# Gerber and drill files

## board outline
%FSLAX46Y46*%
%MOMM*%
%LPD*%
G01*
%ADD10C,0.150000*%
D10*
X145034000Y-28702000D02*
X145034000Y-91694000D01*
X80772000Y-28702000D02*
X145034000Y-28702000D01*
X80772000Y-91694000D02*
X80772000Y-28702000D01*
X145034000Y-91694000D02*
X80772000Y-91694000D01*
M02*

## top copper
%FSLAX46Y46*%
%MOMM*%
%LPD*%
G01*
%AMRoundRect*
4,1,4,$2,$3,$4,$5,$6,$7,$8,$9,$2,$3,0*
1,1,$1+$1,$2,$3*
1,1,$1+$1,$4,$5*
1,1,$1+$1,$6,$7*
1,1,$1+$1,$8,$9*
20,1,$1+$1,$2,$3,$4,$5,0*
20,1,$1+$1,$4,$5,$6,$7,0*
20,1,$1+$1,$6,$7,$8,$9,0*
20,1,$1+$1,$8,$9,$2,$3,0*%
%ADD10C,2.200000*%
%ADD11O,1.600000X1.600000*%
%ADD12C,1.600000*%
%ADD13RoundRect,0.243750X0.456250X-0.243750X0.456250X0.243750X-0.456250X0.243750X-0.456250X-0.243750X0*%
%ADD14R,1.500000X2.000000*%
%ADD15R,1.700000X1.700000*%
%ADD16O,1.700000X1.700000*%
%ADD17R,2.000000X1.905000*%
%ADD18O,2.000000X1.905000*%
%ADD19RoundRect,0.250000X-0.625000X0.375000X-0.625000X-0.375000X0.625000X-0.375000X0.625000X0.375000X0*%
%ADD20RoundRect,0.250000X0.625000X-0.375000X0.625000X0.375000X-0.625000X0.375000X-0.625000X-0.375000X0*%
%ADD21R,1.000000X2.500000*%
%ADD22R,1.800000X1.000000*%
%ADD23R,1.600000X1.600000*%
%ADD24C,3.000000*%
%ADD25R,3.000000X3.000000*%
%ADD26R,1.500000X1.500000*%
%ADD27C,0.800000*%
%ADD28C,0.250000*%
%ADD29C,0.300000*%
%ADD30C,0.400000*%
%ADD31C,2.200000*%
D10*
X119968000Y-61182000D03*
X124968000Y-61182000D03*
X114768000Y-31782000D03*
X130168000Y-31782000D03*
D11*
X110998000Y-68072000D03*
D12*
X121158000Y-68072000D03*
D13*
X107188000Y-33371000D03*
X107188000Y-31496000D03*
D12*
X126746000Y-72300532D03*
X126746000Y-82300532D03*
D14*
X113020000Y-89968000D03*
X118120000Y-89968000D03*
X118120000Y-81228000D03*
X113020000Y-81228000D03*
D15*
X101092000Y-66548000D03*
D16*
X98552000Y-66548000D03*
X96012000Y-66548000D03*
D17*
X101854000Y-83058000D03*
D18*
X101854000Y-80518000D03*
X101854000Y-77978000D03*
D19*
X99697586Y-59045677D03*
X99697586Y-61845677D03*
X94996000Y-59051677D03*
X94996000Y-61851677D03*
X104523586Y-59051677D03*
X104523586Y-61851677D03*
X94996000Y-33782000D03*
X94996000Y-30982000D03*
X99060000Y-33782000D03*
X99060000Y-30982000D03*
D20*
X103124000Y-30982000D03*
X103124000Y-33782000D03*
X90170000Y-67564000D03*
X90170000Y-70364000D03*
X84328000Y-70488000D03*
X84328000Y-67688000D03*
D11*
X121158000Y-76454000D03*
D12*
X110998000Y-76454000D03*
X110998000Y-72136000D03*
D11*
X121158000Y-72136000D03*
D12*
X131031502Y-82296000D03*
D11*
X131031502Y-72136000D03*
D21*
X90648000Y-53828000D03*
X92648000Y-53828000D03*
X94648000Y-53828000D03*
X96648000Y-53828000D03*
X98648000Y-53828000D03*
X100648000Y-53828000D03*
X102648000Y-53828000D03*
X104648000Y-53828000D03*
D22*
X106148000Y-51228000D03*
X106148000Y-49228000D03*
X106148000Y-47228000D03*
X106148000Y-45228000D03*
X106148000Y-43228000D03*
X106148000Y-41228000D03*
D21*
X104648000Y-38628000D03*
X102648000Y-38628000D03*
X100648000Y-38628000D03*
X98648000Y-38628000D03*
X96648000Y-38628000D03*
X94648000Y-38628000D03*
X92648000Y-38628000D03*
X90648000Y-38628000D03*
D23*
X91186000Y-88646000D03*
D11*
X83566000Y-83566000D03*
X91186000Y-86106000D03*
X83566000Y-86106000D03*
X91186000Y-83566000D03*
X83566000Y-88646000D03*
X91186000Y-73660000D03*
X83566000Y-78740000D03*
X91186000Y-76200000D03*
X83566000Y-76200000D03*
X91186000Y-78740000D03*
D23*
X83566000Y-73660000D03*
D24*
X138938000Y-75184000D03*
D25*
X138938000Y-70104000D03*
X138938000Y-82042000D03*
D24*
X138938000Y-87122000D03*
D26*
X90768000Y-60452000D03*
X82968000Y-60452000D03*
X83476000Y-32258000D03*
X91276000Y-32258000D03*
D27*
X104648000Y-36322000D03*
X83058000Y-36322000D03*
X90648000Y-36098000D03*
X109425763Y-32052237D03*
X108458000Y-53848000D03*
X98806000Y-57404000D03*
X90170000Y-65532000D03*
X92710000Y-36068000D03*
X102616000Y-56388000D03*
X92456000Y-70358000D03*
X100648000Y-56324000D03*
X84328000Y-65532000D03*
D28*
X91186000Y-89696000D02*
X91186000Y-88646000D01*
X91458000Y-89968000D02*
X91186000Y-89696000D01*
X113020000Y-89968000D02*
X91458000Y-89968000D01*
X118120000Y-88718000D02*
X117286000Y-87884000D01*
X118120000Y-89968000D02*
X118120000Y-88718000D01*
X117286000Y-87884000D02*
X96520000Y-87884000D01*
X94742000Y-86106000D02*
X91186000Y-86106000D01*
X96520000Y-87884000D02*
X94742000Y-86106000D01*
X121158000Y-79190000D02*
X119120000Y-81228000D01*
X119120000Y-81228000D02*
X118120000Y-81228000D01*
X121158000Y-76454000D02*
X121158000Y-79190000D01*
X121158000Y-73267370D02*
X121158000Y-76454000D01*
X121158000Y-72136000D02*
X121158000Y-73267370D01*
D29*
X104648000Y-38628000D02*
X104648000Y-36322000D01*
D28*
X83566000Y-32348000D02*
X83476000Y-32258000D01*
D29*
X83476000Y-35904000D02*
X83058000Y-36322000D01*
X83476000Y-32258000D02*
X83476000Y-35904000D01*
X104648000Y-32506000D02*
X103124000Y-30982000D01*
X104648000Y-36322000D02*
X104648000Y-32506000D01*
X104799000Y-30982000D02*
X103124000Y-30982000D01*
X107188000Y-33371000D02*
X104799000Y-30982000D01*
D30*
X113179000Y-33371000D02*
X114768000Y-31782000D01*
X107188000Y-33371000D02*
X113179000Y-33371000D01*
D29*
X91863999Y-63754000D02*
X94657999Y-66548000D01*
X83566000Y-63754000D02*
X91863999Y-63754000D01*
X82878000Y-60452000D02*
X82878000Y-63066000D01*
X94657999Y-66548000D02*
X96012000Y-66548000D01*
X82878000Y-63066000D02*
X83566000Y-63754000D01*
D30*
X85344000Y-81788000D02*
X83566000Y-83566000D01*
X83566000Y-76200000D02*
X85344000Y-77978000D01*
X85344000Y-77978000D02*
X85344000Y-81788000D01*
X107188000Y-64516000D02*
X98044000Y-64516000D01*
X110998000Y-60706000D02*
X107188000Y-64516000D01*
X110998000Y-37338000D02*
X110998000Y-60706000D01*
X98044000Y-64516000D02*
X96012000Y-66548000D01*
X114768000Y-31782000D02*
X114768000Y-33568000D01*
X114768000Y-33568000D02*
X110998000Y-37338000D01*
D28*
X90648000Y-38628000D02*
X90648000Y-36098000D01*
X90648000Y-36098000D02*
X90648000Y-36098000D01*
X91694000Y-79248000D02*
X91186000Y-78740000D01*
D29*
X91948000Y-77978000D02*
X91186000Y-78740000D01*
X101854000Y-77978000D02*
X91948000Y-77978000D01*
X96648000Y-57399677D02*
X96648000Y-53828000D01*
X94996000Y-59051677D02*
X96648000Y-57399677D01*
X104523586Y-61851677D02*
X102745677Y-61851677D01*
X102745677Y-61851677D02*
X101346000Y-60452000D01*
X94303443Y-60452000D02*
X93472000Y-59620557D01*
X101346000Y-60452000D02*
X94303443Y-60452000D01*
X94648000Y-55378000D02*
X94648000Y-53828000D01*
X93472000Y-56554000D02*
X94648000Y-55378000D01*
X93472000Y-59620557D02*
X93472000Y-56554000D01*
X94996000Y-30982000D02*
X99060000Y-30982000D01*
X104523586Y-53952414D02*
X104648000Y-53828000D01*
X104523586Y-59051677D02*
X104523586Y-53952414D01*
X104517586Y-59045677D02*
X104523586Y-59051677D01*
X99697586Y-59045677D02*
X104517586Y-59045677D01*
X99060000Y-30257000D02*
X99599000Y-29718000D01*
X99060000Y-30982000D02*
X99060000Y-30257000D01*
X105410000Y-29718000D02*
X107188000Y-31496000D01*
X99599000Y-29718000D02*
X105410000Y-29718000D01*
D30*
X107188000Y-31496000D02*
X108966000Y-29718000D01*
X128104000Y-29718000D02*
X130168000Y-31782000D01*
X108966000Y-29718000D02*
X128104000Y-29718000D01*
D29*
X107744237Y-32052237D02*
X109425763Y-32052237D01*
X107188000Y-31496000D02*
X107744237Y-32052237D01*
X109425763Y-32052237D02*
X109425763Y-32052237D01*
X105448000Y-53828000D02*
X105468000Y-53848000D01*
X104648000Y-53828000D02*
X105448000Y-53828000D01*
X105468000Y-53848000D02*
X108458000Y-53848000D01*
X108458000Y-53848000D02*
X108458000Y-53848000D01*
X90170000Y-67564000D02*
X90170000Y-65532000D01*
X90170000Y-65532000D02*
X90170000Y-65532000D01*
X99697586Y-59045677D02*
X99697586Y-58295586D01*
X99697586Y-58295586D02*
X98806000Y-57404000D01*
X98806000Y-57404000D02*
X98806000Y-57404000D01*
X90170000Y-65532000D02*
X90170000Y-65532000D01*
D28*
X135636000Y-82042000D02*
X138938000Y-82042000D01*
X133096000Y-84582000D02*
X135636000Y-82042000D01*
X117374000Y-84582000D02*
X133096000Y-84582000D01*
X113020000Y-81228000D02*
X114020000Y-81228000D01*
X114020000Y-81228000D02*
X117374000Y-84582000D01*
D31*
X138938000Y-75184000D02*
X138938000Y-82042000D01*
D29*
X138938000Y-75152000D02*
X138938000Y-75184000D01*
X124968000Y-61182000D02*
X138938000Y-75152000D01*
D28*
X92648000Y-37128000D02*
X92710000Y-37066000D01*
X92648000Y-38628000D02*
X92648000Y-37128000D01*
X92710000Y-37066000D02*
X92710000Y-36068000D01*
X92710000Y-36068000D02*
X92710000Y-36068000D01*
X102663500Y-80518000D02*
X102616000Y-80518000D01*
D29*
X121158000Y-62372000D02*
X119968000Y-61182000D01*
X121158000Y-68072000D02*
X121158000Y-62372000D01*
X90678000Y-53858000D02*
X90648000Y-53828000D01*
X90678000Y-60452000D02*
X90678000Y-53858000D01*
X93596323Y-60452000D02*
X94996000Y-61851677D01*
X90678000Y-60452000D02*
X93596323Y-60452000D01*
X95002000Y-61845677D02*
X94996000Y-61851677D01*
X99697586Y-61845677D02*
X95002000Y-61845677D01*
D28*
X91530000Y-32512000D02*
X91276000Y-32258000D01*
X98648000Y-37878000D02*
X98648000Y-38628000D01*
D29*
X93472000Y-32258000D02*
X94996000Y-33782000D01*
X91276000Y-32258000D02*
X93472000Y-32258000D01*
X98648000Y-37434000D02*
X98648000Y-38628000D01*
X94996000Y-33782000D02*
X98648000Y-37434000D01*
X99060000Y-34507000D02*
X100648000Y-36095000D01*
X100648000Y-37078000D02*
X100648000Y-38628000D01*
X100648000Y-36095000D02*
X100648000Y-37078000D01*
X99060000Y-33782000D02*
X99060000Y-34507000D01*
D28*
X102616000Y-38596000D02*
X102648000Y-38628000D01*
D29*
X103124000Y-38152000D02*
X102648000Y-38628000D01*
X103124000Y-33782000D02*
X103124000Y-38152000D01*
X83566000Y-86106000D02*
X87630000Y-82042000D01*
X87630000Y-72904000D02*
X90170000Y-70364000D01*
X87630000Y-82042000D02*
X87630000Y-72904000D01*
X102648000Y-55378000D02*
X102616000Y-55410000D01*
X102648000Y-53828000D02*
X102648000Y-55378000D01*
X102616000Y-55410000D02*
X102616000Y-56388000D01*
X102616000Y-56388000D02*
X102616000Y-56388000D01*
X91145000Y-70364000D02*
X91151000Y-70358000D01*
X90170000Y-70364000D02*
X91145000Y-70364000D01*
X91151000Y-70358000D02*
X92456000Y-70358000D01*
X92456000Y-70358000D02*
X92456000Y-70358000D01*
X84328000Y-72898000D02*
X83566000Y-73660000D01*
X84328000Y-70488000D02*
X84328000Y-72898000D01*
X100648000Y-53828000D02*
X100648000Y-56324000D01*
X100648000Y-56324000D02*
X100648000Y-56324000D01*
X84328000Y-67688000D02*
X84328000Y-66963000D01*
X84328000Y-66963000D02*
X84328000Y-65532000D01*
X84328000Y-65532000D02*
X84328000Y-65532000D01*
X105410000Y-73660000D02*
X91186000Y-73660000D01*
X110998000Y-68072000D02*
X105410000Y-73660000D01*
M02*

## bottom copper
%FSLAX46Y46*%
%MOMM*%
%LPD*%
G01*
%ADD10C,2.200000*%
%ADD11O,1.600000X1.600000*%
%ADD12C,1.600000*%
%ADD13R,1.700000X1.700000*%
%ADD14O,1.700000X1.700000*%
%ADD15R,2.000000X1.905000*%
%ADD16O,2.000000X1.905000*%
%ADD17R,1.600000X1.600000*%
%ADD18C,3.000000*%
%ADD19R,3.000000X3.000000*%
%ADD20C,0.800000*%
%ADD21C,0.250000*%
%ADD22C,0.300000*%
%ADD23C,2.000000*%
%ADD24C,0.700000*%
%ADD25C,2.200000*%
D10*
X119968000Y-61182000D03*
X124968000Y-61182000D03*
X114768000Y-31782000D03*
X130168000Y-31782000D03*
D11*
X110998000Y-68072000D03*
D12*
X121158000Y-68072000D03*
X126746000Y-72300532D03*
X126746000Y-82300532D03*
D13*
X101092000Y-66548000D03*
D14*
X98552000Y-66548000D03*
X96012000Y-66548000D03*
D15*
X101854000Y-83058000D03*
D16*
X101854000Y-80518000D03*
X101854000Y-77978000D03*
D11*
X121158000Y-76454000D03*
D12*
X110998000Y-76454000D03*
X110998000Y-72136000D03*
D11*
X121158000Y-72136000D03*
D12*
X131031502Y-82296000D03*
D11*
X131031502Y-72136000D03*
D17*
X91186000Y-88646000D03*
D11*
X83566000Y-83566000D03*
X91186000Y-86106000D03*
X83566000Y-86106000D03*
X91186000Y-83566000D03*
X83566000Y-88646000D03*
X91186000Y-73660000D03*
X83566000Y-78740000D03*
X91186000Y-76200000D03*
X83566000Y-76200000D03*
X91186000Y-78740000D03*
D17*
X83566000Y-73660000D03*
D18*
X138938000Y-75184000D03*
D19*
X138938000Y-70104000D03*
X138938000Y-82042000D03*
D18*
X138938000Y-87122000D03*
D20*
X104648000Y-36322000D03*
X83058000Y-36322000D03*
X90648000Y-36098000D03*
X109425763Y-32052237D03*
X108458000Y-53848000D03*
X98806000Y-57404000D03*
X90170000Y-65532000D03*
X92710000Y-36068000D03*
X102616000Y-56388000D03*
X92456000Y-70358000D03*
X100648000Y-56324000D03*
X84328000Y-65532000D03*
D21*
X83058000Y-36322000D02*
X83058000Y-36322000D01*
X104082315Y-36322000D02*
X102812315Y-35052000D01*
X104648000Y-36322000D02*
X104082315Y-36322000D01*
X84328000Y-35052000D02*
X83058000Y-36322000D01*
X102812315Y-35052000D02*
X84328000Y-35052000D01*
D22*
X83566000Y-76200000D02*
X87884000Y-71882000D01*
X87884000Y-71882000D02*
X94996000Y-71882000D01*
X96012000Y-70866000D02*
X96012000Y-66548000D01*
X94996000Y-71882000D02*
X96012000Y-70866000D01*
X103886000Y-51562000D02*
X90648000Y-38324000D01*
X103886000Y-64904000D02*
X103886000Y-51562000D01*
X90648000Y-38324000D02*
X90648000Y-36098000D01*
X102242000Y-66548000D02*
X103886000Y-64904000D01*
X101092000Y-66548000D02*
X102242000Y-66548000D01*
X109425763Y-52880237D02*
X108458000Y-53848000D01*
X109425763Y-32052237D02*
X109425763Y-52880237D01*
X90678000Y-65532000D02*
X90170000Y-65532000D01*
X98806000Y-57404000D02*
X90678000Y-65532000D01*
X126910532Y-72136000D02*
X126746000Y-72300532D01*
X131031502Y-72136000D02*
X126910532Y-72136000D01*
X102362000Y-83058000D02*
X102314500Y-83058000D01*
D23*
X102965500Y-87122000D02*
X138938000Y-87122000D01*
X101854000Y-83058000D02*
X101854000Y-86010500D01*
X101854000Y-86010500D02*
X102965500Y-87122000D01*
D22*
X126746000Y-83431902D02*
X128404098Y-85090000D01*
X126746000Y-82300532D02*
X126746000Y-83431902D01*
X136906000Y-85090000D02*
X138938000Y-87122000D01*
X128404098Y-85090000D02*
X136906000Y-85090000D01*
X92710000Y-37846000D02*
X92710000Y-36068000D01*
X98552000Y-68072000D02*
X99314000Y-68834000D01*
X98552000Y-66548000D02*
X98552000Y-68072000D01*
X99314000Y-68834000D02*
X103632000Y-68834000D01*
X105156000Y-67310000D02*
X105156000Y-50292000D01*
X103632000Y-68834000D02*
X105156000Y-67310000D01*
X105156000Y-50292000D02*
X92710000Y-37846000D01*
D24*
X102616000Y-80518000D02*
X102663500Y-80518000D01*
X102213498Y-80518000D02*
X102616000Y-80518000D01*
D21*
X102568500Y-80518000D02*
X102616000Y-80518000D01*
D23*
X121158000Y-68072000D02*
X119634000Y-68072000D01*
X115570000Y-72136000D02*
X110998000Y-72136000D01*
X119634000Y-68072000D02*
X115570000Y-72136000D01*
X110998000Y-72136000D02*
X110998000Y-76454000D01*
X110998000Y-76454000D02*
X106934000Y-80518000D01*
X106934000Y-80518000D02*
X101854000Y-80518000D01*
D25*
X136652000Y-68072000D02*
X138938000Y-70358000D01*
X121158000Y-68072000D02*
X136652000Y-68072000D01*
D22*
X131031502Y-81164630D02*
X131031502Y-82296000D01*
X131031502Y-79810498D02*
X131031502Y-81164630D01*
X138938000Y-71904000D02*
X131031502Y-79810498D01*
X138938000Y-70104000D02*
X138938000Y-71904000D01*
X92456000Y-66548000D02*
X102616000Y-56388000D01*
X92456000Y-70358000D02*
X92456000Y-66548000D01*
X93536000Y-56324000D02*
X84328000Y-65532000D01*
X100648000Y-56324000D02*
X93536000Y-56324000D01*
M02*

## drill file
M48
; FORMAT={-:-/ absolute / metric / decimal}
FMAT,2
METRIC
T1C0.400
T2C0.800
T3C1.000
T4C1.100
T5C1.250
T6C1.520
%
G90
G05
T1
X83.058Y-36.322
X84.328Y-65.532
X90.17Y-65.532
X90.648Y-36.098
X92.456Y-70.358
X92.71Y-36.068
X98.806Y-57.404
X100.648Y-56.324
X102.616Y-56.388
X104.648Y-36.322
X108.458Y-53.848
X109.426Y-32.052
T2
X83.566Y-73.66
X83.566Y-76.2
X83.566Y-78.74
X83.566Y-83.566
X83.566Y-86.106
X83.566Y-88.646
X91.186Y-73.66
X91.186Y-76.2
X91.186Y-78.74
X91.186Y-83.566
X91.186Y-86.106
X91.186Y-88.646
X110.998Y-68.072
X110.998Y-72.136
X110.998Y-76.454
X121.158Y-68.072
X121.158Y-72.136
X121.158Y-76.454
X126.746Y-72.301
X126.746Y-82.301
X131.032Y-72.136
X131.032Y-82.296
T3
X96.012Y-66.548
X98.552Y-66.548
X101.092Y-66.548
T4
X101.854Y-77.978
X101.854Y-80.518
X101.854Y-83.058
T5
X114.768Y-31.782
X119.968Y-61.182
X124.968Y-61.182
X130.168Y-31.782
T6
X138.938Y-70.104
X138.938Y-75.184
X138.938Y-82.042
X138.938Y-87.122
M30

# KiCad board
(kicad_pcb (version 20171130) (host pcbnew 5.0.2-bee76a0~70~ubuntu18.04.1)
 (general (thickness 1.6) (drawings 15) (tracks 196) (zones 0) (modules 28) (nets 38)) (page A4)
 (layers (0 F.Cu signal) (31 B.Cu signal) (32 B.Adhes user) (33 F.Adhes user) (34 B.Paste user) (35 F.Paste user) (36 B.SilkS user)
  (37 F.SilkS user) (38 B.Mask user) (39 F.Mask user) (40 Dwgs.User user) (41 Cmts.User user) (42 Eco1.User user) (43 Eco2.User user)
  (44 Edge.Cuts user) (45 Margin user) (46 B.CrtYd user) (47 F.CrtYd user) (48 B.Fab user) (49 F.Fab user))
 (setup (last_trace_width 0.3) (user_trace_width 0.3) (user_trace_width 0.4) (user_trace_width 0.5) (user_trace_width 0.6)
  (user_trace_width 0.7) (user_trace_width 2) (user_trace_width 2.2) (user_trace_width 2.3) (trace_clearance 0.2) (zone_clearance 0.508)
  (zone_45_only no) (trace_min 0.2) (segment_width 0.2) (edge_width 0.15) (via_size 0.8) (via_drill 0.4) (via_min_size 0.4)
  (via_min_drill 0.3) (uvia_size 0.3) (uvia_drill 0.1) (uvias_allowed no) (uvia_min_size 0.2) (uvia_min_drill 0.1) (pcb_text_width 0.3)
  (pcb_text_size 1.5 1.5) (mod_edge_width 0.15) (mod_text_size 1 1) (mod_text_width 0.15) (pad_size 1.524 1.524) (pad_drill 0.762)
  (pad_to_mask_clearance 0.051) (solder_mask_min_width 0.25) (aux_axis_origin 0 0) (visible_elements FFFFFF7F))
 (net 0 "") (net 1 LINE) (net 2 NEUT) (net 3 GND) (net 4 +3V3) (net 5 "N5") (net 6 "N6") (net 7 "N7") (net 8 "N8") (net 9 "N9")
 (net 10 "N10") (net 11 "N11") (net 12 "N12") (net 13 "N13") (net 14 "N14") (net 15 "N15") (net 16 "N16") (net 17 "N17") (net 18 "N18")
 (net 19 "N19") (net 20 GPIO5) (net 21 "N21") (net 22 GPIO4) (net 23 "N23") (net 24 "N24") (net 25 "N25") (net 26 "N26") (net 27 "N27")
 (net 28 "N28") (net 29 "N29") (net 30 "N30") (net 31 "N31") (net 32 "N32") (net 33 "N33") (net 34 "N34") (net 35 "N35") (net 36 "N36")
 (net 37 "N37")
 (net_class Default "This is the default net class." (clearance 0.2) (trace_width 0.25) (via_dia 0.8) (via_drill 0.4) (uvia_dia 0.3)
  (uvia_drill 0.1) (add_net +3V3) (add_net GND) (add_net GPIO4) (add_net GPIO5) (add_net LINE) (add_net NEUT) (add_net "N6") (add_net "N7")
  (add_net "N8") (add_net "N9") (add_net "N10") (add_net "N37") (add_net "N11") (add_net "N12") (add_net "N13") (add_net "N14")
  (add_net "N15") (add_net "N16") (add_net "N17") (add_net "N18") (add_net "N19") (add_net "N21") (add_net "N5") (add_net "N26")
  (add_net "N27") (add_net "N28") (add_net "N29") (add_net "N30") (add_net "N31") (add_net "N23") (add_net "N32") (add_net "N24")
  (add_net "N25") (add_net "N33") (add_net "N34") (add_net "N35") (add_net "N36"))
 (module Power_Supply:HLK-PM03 (layer F.Cu) (at 122.468 46.482 90)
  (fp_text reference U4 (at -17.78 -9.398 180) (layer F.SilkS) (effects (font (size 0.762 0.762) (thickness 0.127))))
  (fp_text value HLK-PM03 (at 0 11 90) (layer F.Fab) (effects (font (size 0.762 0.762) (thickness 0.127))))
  (pad 1 thru_hole circle (at -14.7 -2.5 90) (size 2.2 2.2) (drill 1.25) (layers *.Cu *.Mask) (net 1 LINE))
  (pad 2 thru_hole circle (at -14.7 2.5 90) (size 2.2 2.2) (drill 1.25) (layers *.Cu *.Mask) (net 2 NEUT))
  (pad 3 thru_hole circle (at 14.7 -7.7 90) (size 2.2 2.2) (drill 1.25) (layers *.Cu *.Mask) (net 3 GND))
  (pad 4 thru_hole circle (at 14.7 7.7 90) (size 2.2 2.2) (drill 1.25) (layers *.Cu *.Mask) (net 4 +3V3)))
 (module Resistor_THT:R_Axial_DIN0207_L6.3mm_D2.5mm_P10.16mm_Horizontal (layer F.Cu) (at 121.158 68.072 180)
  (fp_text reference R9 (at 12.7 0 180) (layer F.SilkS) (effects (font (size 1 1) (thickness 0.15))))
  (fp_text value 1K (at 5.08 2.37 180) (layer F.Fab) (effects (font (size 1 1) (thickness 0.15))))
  (pad 2 thru_hole oval (at 10.16 0 180) (size 1.6 1.6) (drill 0.8) (layers *.Cu *.Mask) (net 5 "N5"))
  (pad 1 thru_hole circle (at 0 0 180) (size 1.6 1.6) (drill 0.8) (layers *.Cu *.Mask) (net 1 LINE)))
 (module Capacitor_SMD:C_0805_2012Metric (layer F.Cu) (at 107.188 32.4335 90)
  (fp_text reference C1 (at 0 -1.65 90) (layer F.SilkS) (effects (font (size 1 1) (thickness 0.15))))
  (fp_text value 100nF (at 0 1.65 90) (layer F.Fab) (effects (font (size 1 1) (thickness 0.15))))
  (pad 1 smd roundrect (at -0.9375 0 90) (size 0.975 1.4) (layers F.Cu F.Paste F.Mask) (roundrect_rratio 0.25) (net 3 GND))
  (pad 2 smd roundrect (at 0.9375 0 90) (size 0.975 1.4) (layers F.Cu F.Paste F.Mask) (roundrect_rratio 0.25) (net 4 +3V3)))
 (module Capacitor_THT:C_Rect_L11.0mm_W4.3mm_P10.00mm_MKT (layer F.Cu) (at 126.746 72.300532 270)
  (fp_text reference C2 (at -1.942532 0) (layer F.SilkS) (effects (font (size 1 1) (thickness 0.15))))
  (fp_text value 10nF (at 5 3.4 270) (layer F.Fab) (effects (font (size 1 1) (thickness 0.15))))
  (pad 1 thru_hole circle (at 0 0 270) (size 1.6 1.6) (drill 0.8) (layers *.Cu *.Mask) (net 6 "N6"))
  (pad 2 thru_hole circle (at 10 0 270) (size 1.6 1.6) (drill 0.8) (layers *.Cu *.Mask) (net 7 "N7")))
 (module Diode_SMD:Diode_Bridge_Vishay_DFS (layer F.Cu) (at 115.57 85.598 90)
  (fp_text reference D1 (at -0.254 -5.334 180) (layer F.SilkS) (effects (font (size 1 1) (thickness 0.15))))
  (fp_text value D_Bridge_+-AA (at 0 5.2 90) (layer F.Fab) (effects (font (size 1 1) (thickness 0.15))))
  (pad 1 smd rect (at -4.37 -2.55 90) (size 2 1.5) (layers F.Cu F.Paste F.Mask) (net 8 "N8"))
  (pad 2 smd rect (at -4.37 2.55 90) (size 2 1.5) (layers F.Cu F.Paste F.Mask) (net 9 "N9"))
  (pad 3 smd rect (at 4.37 2.55 90) (size 2 1.5) (layers F.Cu F.Paste F.Mask) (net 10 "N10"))
  (pad 4 smd rect (at 4.37 -2.55 90) (size 2 1.5) (layers F.Cu F.Paste F.Mask) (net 2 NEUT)))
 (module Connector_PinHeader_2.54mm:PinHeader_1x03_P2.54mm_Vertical (layer F.Cu) (at 101.092 66.548 270)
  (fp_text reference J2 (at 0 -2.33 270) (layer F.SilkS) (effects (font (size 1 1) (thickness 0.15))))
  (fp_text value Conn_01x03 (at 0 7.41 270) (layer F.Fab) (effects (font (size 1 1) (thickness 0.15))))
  (pad 1 thru_hole rect (at 0 0 270) (size 1.7 1.7) (drill 1) (layers *.Cu *.Mask) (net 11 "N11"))
  (pad 2 thru_hole oval (at 0 2.54 270) (size 1.7 1.7) (drill 1) (layers *.Cu *.Mask) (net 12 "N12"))
  (pad 3 thru_hole oval (at 0 5.08 270) (size 1.7 1.7) (drill 1) (layers *.Cu *.Mask) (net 3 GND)))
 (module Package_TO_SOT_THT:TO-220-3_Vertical (layer F.Cu) (at 101.854 83.058 90)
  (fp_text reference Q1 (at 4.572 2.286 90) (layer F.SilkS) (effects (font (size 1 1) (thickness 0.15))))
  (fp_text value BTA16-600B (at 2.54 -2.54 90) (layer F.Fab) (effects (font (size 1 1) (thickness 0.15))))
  (pad 1 thru_hole rect (at 0 0 90) (size 1.905 2) (drill 1.1) (layers *.Cu *.Mask) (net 7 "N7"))
  (pad 2 thru_hole oval (at 2.54 0 90) (size 1.905 2) (drill 1.1) (layers *.Cu *.Mask) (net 1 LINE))
  (pad 3 thru_hole oval (at 5.08 0 90) (size 1.905 2) (drill 1.1) (layers *.Cu *.Mask) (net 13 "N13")))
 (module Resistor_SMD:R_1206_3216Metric (layer F.Cu) (at 99.697586 60.445677 270)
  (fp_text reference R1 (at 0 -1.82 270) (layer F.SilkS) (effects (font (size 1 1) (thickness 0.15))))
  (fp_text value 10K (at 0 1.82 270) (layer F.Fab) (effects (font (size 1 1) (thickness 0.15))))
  (pad 1 smd roundrect (at -1.4 0 270) (size 1.25 1.75) (layers F.Cu F.Paste F.Mask) (roundrect_rratio 0.2) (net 4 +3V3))
  (pad 2 smd roundrect (at 1.4 0 270) (size 1.25 1.75) (layers F.Cu F.Paste F.Mask) (roundrect_rratio 0.2) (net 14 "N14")))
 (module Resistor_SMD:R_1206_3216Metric (layer F.Cu) (at 94.996 60.451677 270)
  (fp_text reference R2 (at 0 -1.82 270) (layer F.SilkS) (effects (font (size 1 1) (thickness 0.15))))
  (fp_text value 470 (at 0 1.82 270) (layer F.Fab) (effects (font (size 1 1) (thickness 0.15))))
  (pad 1 smd roundrect (at -1.4 0 270) (size 1.25 1.75) (layers F.Cu F.Paste F.Mask) (roundrect_rratio 0.2) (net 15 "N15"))
  (pad 2 smd roundrect (at 1.4 0 270) (size 1.25 1.75) (layers F.Cu F.Paste F.Mask) (roundrect_rratio 0.2) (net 14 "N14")))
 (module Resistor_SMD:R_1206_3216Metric (layer F.Cu) (at 104.523586 60.451677 270)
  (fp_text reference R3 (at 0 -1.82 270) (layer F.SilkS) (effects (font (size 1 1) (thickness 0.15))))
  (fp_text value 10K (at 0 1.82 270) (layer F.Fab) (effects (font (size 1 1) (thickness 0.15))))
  (pad 1 smd roundrect (at -1.4 0 270) (size 1.25 1.75) (layers F.Cu F.Paste F.Mask) (roundrect_rratio 0.2) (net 4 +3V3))
  (pad 2 smd roundrect (at 1.4 0 270) (size 1.25 1.75) (layers F.Cu F.Paste F.Mask) (roundrect_rratio 0.2) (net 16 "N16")))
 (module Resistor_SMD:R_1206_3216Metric (layer F.Cu) (at 94.996 32.382 270)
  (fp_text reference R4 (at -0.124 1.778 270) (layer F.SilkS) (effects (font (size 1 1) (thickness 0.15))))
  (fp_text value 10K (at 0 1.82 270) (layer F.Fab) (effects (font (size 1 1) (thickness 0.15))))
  (pad 2 smd roundrect (at 1.4 0 270) (size 1.25 1.75) (layers F.Cu F.Paste F.Mask) (roundrect_rratio 0.2) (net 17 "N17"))
  (pad 1 smd roundrect (at -1.4 0 270) (size 1.25 1.75) (layers F.Cu F.Paste F.Mask) (roundrect_rratio 0.2) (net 4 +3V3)))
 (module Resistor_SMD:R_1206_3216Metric (layer F.Cu) (at 99.06 32.382 270)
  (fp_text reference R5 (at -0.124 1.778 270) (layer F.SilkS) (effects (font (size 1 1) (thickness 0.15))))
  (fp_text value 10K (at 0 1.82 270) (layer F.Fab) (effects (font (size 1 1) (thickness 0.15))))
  (pad 2 smd roundrect (at 1.4 0 270) (size 1.25 1.75) (layers F.Cu F.Paste F.Mask) (roundrect_rratio 0.2) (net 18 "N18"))
  (pad 1 smd roundrect (at -1.4 0 270) (size 1.25 1.75) (layers F.Cu F.Paste F.Mask) (roundrect_rratio 0.2) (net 4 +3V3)))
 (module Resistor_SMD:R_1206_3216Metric (layer F.Cu) (at 103.124 32.382 90)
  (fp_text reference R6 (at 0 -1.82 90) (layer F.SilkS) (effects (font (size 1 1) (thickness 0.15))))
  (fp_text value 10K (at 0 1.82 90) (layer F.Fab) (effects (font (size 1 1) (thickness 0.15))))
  (pad 2 smd roundrect (at 1.4 0 90) (size 1.25 1.75) (layers F.Cu F.Paste F.Mask) (roundrect_rratio 0.2) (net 3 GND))
  (pad 1 smd roundrect (at -1.4 0 90) (size 1.25 1.75) (layers F.Cu F.Paste F.Mask) (roundrect_rratio 0.2) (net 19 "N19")))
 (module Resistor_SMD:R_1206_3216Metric (layer F.Cu) (at 90.17 68.964 90)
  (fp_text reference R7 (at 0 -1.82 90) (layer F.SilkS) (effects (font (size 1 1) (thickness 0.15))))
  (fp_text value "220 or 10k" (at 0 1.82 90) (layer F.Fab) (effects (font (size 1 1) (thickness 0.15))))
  (pad 2 smd roundrect (at 1.4 0 90) (size 1.25 1.75) (layers F.Cu F.Paste F.Mask) (roundrect_rratio 0.2) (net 4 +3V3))
  (pad 1 smd roundrect (at -1.4 0 90) (size 1.25 1.75) (layers F.Cu F.Paste F.Mask) (roundrect_rratio 0.2) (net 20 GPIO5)))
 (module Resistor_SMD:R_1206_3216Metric (layer F.Cu) (at 84.328 69.088 90)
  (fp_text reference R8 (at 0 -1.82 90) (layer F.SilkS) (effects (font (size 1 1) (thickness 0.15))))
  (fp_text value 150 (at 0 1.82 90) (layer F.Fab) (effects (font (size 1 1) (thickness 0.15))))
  (pad 1 smd roundrect (at -1.4 0 90) (size 1.25 1.75) (layers F.Cu F.Paste F.Mask) (roundrect_rratio 0.2) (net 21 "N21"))
  (pad 2 smd roundrect (at 1.4 0 90) (size 1.25 1.75) (layers F.Cu F.Paste F.Mask) (roundrect_rratio 0.2) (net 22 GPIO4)))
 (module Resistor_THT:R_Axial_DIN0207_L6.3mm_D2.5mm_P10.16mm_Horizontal (layer F.Cu) (at 110.998 76.454)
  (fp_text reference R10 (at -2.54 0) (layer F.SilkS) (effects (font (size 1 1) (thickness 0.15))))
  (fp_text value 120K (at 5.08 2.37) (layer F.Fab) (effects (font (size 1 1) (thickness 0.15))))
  (pad 2 thru_hole oval (at 10.16 0) (size 1.6 1.6) (drill 0.8) (layers *.Cu *.Mask) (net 10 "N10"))
  (pad 1 thru_hole circle (at 0 0) (size 1.6 1.6) (drill 0.8) (layers *.Cu *.Mask) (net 1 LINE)))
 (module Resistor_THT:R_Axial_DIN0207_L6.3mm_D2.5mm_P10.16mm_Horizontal (layer F.Cu) (at 110.998 72.136)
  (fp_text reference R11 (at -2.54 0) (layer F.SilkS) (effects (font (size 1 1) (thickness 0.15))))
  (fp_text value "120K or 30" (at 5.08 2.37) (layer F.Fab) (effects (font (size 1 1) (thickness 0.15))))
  (pad 1 thru_hole circle (at 0 0) (size 1.6 1.6) (drill 0.8) (layers *.Cu *.Mask) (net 1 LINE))
  (pad 2 thru_hole oval (at 10.16 0) (size 1.6 1.6) (drill 0.8) (layers *.Cu *.Mask) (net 10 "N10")))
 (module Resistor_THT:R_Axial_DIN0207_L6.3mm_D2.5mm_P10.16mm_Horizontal (layer F.Cu) (at 131.031502 82.296 90)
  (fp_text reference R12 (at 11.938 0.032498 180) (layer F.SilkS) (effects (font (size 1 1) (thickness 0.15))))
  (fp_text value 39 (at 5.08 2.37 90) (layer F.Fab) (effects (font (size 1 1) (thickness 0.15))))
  (pad 1 thru_hole circle (at 0 0 90) (size 1.6 1.6) (drill 0.8) (layers *.Cu *.Mask) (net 1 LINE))
  (pad 2 thru_hole oval (at 10.16 0 90) (size 1.6 1.6) (drill 0.8) (layers *.Cu *.Mask) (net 6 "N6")))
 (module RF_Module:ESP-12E (layer F.Cu) (at 94.148 46.228 90)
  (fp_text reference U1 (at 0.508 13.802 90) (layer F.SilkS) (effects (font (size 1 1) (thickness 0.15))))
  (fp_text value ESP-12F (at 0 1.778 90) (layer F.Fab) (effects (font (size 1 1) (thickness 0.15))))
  (pad 1 smd rect (at -7.6 -3.5 90) (size 2.5 1) (layers F.Cu F.Paste F.Mask) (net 14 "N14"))
  (pad 2 smd rect (at -7.6 -1.5 90) (size 2.5 1) (layers F.Cu F.Paste F.Mask) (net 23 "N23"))
  (pad 3 smd rect (at -7.6 0.5 90) (size 2.5 1) (layers F.Cu F.Paste F.Mask) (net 16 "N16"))
  (pad 4 smd rect (at -7.6 2.5 90) (size 2.5 1) (layers F.Cu F.Paste F.Mask) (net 15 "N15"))
  (pad 5 smd rect (at -7.6 4.5 90) (size 2.5 1) (layers F.Cu F.Paste F.Mask) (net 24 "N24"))
  (pad 6 smd rect (at -7.6 6.5 90) (size 2.5 1) (layers F.Cu F.Paste F.Mask) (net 22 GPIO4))
  (pad 7 smd rect (at -7.6 8.5 90) (size 2.5 1) (layers F.Cu F.Paste F.Mask) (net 20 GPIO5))
  (pad 8 smd rect (at -7.6 10.5 90) (size 2.5 1) (layers F.Cu F.Paste F.Mask) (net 4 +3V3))
  (pad 9 smd rect (at -5 12 90) (size 1 1.8) (layers F.Cu F.Paste F.Mask) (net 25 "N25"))
  (pad 10 smd rect (at -3 12 90) (size 1 1.8) (layers F.Cu F.Paste F.Mask) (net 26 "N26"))
  (pad 11 smd rect (at -1 12 90) (size 1 1.8) (layers F.Cu F.Paste F.Mask) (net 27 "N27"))
  (pad 12 smd rect (at 1 12 90) (size 1 1.8) (layers F.Cu F.Paste F.Mask) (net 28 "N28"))
  (pad 13 smd rect (at 3 12 90) (size 1 1.8) (layers F.Cu F.Paste F.Mask) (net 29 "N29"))
  (pad 14 smd rect (at 5 12 90) (size 1 1.8) (layers F.Cu F.Paste F.Mask) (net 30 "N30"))
  (pad 15 smd rect (at 7.6 10.5 90) (size 2.5 1) (layers F.Cu F.Paste F.Mask) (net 3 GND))
  (pad 16 smd rect (at 7.6 8.5 90) (size 2.5 1) (layers F.Cu F.Paste F.Mask) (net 19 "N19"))
  (pad 17 smd rect (at 7.6 6.5 90) (size 2.5 1) (layers F.Cu F.Paste F.Mask) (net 18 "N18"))
  (pad 18 smd rect (at 7.6 4.5 90) (size 2.5 1) (layers F.Cu F.Paste F.Mask) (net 17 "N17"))
  (pad 19 smd rect (at 7.6 2.5 90) (size 2.5 1) (layers F.Cu F.Paste F.Mask) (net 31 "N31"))
  (pad 20 smd rect (at 7.6 0.5 90) (size 2.5 1) (layers F.Cu F.Paste F.Mask) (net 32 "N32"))
  (pad 21 smd rect (at 7.6 -1.5 90) (size 2.5 1) (layers F.Cu F.Paste F.Mask) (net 12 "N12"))
  (pad 22 smd rect (at 7.6 -3.5 90) (size 2.5 1) (layers F.Cu F.Paste F.Mask) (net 11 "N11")))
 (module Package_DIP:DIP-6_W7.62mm (layer F.Cu) (at 91.186 88.646 180)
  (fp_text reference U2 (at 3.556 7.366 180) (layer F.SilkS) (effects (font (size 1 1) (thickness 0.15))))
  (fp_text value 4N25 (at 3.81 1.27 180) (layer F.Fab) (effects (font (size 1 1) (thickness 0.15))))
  (pad 1 thru_hole rect (at 0 0 180) (size 1.6 1.6) (drill 0.8) (layers *.Cu *.Mask) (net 8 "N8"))
  (pad 4 thru_hole oval (at 7.62 5.08 180) (size 1.6 1.6) (drill 0.8) (layers *.Cu *.Mask) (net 3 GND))
  (pad 2 thru_hole oval (at 0 2.54 180) (size 1.6 1.6) (drill 0.8) (layers *.Cu *.Mask) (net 9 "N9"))
  (pad 5 thru_hole oval (at 7.62 2.54 180) (size 1.6 1.6) (drill 0.8) (layers *.Cu *.Mask) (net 20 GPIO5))
  (pad 3 thru_hole oval (at 0 5.08 180) (size 1.6 1.6) (drill 0.8) (layers *.Cu *.Mask) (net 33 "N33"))
  (pad 6 thru_hole oval (at 7.62 0 180) (size 1.6 1.6) (drill 0.8) (layers *.Cu *.Mask) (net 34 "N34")))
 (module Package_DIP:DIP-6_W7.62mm (layer F.Cu) (at 83.566 73.66)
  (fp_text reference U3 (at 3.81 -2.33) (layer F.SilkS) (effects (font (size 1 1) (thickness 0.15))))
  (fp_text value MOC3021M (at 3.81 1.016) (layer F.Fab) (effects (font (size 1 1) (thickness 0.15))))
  (pad 6 thru_hole oval (at 7.62 0) (size 1.6 1.6) (drill 0.8) (layers *.Cu *.Mask) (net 5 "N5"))
  (pad 3 thru_hole oval (at 0 5.08) (size 1.6 1.6) (drill 0.8) (layers *.Cu *.Mask) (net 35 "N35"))
  (pad 5 thru_hole oval (at 7.62 2.54) (size 1.6 1.6) (drill 0.8) (layers *.Cu *.Mask) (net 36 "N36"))
  (pad 2 thru_hole oval (at 0 2.54) (size 1.6 1.6) (drill 0.8) (layers *.Cu *.Mask) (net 3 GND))
  (pad 4 thru_hole oval (at 7.62 5.08) (size 1.6 1.6) (drill 0.8) (layers *.Cu *.Mask) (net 13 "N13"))
  (pad 1 thru_hole rect (at 0 0) (size 1.6 1.6) (drill 0.8) (layers *.Cu *.Mask) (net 21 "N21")))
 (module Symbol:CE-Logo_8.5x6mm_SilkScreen (layer F.Cu) (at 126.238 87.63)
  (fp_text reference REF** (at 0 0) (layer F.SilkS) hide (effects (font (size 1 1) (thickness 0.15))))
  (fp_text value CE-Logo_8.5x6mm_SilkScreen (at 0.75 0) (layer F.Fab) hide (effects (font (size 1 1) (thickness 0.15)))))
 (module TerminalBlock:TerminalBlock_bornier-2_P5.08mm (layer F.Cu) (at 138.938 70.104 270)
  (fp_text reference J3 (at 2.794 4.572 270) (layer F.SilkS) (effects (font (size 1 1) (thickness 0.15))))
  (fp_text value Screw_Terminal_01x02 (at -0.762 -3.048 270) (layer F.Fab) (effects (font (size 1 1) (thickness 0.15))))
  (pad 2 thru_hole circle (at 5.08 0 270) (size 3 3) (drill 1.52) (layers *.Cu *.Mask) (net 2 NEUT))
  (pad 1 thru_hole rect (at 0 0 270) (size 3 3) (drill 1.52) (layers *.Cu *.Mask) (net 1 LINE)))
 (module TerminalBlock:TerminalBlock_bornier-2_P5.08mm (layer F.Cu) (at 138.938 82.042 270)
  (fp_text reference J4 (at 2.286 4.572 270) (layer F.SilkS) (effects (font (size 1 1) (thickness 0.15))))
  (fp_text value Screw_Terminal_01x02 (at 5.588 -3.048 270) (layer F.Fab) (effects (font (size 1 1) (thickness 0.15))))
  (pad 1 thru_hole rect (at 0 0 270) (size 3 3) (drill 1.52) (layers *.Cu *.Mask) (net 2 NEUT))
  (pad 2 thru_hole circle (at 5.08 0 270) (size 3 3) (drill 1.52) (layers *.Cu *.Mask) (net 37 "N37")))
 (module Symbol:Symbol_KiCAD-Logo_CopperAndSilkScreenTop (layer F.Cu) (at 142.494 48.26 90)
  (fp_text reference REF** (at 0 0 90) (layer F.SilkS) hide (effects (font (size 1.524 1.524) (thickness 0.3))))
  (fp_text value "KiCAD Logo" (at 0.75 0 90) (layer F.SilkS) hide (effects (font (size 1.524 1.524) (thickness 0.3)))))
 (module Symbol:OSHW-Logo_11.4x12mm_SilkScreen (layer F.Cu) (at 138.684 35.56 90)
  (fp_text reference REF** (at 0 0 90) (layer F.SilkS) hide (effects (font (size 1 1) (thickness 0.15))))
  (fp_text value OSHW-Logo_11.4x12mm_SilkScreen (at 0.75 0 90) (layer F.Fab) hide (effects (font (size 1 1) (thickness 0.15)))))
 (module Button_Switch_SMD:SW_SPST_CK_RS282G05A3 (layer F.Cu) (at 86.868 60.452)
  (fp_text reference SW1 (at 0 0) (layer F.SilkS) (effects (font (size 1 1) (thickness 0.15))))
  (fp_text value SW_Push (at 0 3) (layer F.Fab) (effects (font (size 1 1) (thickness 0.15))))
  (pad 2 smd rect (at 3.9 0) (size 1.5 1.5) (layers F.Cu F.Paste F.Mask) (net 14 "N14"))
  (pad 1 smd rect (at -3.9 0) (size 1.5 1.5) (layers F.Cu F.Paste F.Mask) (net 3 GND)))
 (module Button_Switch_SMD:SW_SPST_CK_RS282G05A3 (layer F.Cu) (at 87.376 32.258)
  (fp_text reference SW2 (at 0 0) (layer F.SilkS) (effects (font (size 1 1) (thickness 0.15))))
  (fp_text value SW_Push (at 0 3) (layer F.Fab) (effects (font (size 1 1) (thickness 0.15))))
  (pad 1 smd rect (at -3.9 0) (size 1.5 1.5) (layers F.Cu F.Paste F.Mask) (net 3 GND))
  (pad 2 smd rect (at 3.9 0) (size 1.5 1.5) (layers F.Cu F.Paste F.Mask) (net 17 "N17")))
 (gr_line (start 145.034 28.702) (end 145.034 91.694) (layer Edge.Cuts) (width 0.15))
 (gr_line (start 80.772 28.702) (end 145.034 28.702) (layer Edge.Cuts) (width 0.15))
 (gr_line (start 80.772 91.694) (end 80.772 28.702) (layer Edge.Cuts) (width 0.15))
 (gr_line (start 145.034 91.694) (end 80.772 91.694) (layer Edge.Cuts) (width 0.15))
 (segment (start 91.186 89.696) (end 91.186 88.646) (width 0.25) (layer F.Cu) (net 8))
 (segment (start 91.458 89.968) (end 91.186 89.696) (width 0.25) (layer F.Cu) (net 8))
 (segment (start 113.02 89.968) (end 91.458 89.968) (width 0.25) (layer F.Cu) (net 8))
 (segment (start 118.12 88.718) (end 117.286 87.884) (width 0.25) (layer F.Cu) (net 9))
 (segment (start 118.12 89.968) (end 118.12 88.718) (width 0.25) (layer F.Cu) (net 9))
 (segment (start 117.286 87.884) (end 96.52 87.884) (width 0.25) (layer F.Cu) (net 9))
 (segment (start 94.742 86.106) (end 91.186 86.106) (width 0.25) (layer F.Cu) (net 9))
 (segment (start 96.52 87.884) (end 94.742 86.106) (width 0.25) (layer F.Cu) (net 9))
 (segment (start 121.158 79.19) (end 119.12 81.228) (width 0.25) (layer F.Cu) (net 10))
 (segment (start 119.12 81.228) (end 118.12 81.228) (width 0.25) (layer F.Cu) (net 10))
 (segment (start 121.158 76.454) (end 121.158 79.19) (width 0.25) (layer F.Cu) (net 10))
 (segment (start 121.158 73.26737) (end 121.158 76.454) (width 0.25) (layer F.Cu) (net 10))
 (segment (start 121.158 72.136) (end 121.158 73.26737) (width 0.25) (layer F.Cu) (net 10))
 (via (at 104.648 36.322) (size 0.8) (drill 0.4) (layers F.Cu B.Cu) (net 3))
 (segment (start 83.058 36.322) (end 83.058 36.322) (width 0.25) (layer B.Cu) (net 3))
 (via (at 83.058 36.322) (size 0.8) (drill 0.4) (layers F.Cu B.Cu) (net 3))
 (segment (start 104.648 38.628) (end 104.648 36.322) (width 0.3) (layer F.Cu) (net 3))
 (segment (start 83.566 32.348) (end 83.476 32.258) (width 0.25) (layer F.Cu) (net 3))
 (segment (start 83.476 35.904) (end 83.058 36.322) (width 0.3) (layer F.Cu) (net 3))
 (segment (start 83.476 32.258) (end 83.476 35.904) (width 0.3) (layer F.Cu) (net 3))
 (segment (start 104.648 32.506) (end 103.124 30.982) (width 0.3) (layer F.Cu) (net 3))
 (segment (start 104.648 36.322) (end 104.648 32.506) (width 0.3) (layer F.Cu) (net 3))
 (segment (start 104.082315 36.322) (end 102.812315 35.052) (width 0.25) (layer B.Cu) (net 3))
 (segment (start 104.648 36.322) (end 104.082315 36.322) (width 0.25) (layer B.Cu) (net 3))
 (segment (start 84.328 35.052) (end 83.058 36.322) (width 0.25) (layer B.Cu) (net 3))
 (segment (start 102.812315 35.052) (end 84.328 35.052) (width 0.25) (layer B.Cu) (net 3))
 (segment (start 104.799 30.982) (end 103.124 30.982) (width 0.3) (layer F.Cu) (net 3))
 (segment (start 107.188 33.371) (end 104.799 30.982) (width 0.3) (layer F.Cu) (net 3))
 (segment (start 113.179 33.371) (end 114.768 31.782) (width 0.4) (layer F.Cu) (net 3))
 (segment (start 107.188 33.371) (end 113.179 33.371) (width 0.4) (layer F.Cu) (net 3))
 (segment (start 91.863999 63.754) (end 94.657999 66.548) (width 0.3) (layer F.Cu) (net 3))
 (segment (start 83.566 63.754) (end 91.863999 63.754) (width 0.3) (layer F.Cu) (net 3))
 (segment (start 82.878 60.452) (end 82.878 63.066) (width 0.3) (layer F.Cu) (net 3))
 (segment (start 94.657999 66.548) (end 96.012 66.548) (width 0.3) (layer F.Cu) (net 3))
 (segment (start 82.878 63.066) (end 83.566 63.754) (width 0.3) (layer F.Cu) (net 3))
 (segment (start 85.344 81.788) (end 83.566 83.566) (width 0.4) (layer F.Cu) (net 3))
 (segment (start 83.566 76.2) (end 85.344 77.978) (width 0.4) (layer F.Cu) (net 3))
 (segment (start 85.344 77.978) (end 85.344 81.788) (width 0.4) (layer F.Cu) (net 3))
 (segment (start 107.188 64.516) (end 98.044 64.516) (width 0.4) (layer F.Cu) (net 3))
 (segment (start 110.998 60.706) (end 107.188 64.516) (width 0.4) (layer F.Cu) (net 3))
 (segment (start 110.998 37.338) (end 110.998 60.706) (width 0.4) (layer F.Cu) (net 3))
 (segment (start 98.044 64.516) (end 96.012 66.548) (width 0.4) (layer F.Cu) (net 3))
 (segment (start 114.768 31.782) (end 114.768 33.568) (width 0.4) (layer F.Cu) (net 3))
 (segment (start 114.768 33.568) (end 110.998 37.338) (width 0.4) (layer F.Cu) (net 3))
 (segment (start 83.566 76.2) (end 87.884 71.882) (width 0.3) (layer B.Cu) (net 3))
 (segment (start 87.884 71.882) (end 94.996 71.882) (width 0.3) (layer B.Cu) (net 3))
 (segment (start 96.012 70.866) (end 96.012 66.548) (width 0.3) (layer B.Cu) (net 3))
 (segment (start 94.996 71.882) (end 96.012 70.866) (width 0.3) (layer B.Cu) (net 3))
 (segment (start 90.648 38.628) (end 90.648 36.098) (width 0.25) (layer F.Cu) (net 11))
 (segment (start 90.648 36.098) (end 90.648 36.098) (width 0.25) (layer F.Cu) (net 11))
 (via (at 90.648 36.098) (size 0.8) (drill 0.4) (layers F.Cu B.Cu) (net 11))
 (segment (start 103.886 51.562) (end 90.648 38.324) (width 0.3) (layer B.Cu) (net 11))
 (segment (start 103.886 64.904) (end 103.886 51.562) (width 0.3) (layer B.Cu) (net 11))
 (segment (start 90.648 38.324) (end 90.648 36.098) (width 0.3) (layer B.Cu) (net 11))
 (segment (start 102.242 66.548) (end 103.886 64.904) (width 0.3) (layer B.Cu) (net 11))
 (segment (start 101.092 66.548) (end 102.242 66.548) (width 0.3) (layer B.Cu) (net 11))
 (segment (start 91.694 79.248) (end 91.186 78.74) (width 0.25) (layer F.Cu) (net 13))
 (segment (start 91.948 77.978) (end 91.186 78.74) (width 0.3) (layer F.Cu) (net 13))
 (segment (start 101.854 77.978) (end 91.948 77.978) (width 0.3) (layer F.Cu) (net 13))
 (segment (start 96.648 57.399677) (end 96.648 53.828) (width 0.3) (layer F.Cu) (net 15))
 (segment (start 94.996 59.051677) (end 96.648 57.399677) (width 0.3) (layer F.Cu) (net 15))
 (segment (start 104.523586 61.851677) (end 102.745677 61.851677) (width 0.3) (layer F.Cu) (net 16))
 (segment (start 102.745677 61.851677) (end 101.346 60.452) (width 0.3) (layer F.Cu) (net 16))
 (segment (start 94.303443 60.452) (end 93.472 59.620557) (width 0.3) (layer F.Cu) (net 16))
 (segment (start 101.346 60.452) (end 94.303443 60.452) (width 0.3) (layer F.Cu) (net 16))
 (segment (start 94.648 55.378) (end 94.648 53.828) (width 0.3) (layer F.Cu) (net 16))
 (segment (start 93.472 56.554) (end 94.648 55.378) (width 0.3) (layer F.Cu) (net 16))
 (segment (start 93.472 59.620557) (end 93.472 56.554) (width 0.3) (layer F.Cu) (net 16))
 (segment (start 94.996 30.982) (end 99.06 30.982) (width 0.3) (layer F.Cu) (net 4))
 (segment (start 104.523586 53.952414) (end 104.648 53.828) (width 0.3) (layer F.Cu) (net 4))
 (segment (start 104.523586 59.051677) (end 104.523586 53.952414) (width 0.3) (layer F.Cu) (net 4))
 (segment (start 104.517586 59.045677) (end 104.523586 59.051677) (width 0.3) (layer F.Cu) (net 4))
 (segment (start 99.697586 59.045677) (end 104.517586 59.045677) (width 0.3) (layer F.Cu) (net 4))
 (segment (start 99.06 30.257) (end 99.599 29.718) (width 0.3) (layer F.Cu) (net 4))
 (segment (start 99.06 30.982) (end 99.06 30.257) (width 0.3) (layer F.Cu) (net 4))
 (segment (start 105.41 29.718) (end 107.188 31.496) (width 0.3) (layer F.Cu) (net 4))
 (segment (start 99.599 29.718) (end 105.41 29.718) (width 0.3) (layer F.Cu) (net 4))
 (segment (start 107.188 31.496) (end 108.966 29.718) (width 0.4) (layer F.Cu) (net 4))
 (segment (start 128.104 29.718) (end 130.168 31.782) (width 0.4) (layer F.Cu) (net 4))
 (segment (start 108.966 29.718) (end 128.104 29.718) (width 0.4) (layer F.Cu) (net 4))
 (segment (start 107.744237 32.052237) (end 109.425763 32.052237) (width 0.3) (layer F.Cu) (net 4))
 (segment (start 107.188 31.496) (end 107.744237 32.052237) (width 0.3) (layer F.Cu) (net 4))
 (segment (start 109.425763 32.052237) (end 109.425763 32.052237) (width 0.3) (layer F.Cu) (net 4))
 (via (at 109.425763 32.052237) (size 0.8) (drill 0.4) (layers F.Cu B.Cu) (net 4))
 (segment (start 105.448 53.828) (end 105.468 53.848) (width 0.3) (layer F.Cu) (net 4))
 (segment (start 104.648 53.828) (end 105.448 53.828) (width 0.3) (layer F.Cu) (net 4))
 (segment (start 105.468 53.848) (end 108.458 53.848) (width 0.3) (layer F.Cu) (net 4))
 (segment (start 108.458 53.848) (end 108.458 53.848) (width 0.3) (layer F.Cu) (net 4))
 (via (at 108.458 53.848) (size 0.8) (drill 0.4) (layers F.Cu B.Cu) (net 4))
 (segment (start 109.425763 52.880237) (end 108.458 53.848) (width 0.3) (layer B.Cu) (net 4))
 (segment (start 109.425763 32.052237) (end 109.425763 52.880237) (width 0.3) (layer B.Cu) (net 4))
 (segment (start 90.17 67.564) (end 90.17 65.532) (width 0.3) (layer F.Cu) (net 4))
 (segment (start 90.17 65.532) (end 90.17 65.532) (width 0.3) (layer F.Cu) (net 4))
 (segment (start 99.697586 59.045677) (end 99.697586 58.295586) (width 0.3) (layer F.Cu) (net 4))
 (segment (start 99.697586 58.295586) (end 98.806 57.404) (width 0.3) (layer F.Cu) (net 4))
 (segment (start 98.806 57.404) (end 98.806 57.404) (width 0.3) (layer F.Cu) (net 4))
 (via (at 98.806 57.404) (size 0.8) (drill 0.4) (layers F.Cu B.Cu) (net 4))
 (segment (start 90.17 65.532) (end 90.17 65.532) (width 0.3) (layer F.Cu) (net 4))
 (via (at 90.17 65.532) (size 0.8) (drill 0.4) (layers F.Cu B.Cu) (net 4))
 (segment (start 90.678 65.532) (end 90.17 65.532) (width 0.3) (layer B.Cu) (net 4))
 (segment (start 98.806 57.404) (end 90.678 65.532) (width 0.3) (layer B.Cu) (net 4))
 (segment (start 126.910532 72.136) (end 126.746 72.300532) (width 0.3) (layer B.Cu) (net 6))
 (segment (start 131.031502 72.136) (end 126.910532 72.136) (width 0.3) (layer B.Cu) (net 6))
 (segment (start 102.362 83.058) (end 102.3145 83.058) (width 0.3) (layer B.Cu) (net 7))
 (segment (start 102.9655 87.122) (end 138.938 87.122) (width 2) (layer B.Cu) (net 7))
 (segment (start 101.854 83.058) (end 101.854 86.0105) (width 2) (layer B.Cu) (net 7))
 (segment (start 101.854 86.0105) (end 102.9655 87.122) (width 2) (layer B.Cu) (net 7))
 (segment (start 126.746 83.431902) (end 128.404098 85.09) (width 0.3) (layer B.Cu) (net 7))
 (segment (start 126.746 82.300532) (end 126.746 83.431902) (width 0.3) (layer B.Cu) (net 7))
 (segment (start 136.906 85.09) (end 138.938 87.122) (width 0.3) (layer B.Cu) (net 7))
 (segment (start 128.404098 85.09) (end 136.906 85.09) (width 0.3) (layer B.Cu) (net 7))
 (segment (start 135.636 82.042) (end 138.938 82.042) (width 0.25) (layer F.Cu) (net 2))
 (segment (start 133.096 84.582) (end 135.636 82.042) (width 0.25) (layer F.Cu) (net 2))
 (segment (start 117.374 84.582) (end 133.096 84.582) (width 0.25) (layer F.Cu) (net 2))
 (segment (start 113.02 81.228) (end 114.02 81.228) (width 0.25) (layer F.Cu) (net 2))
 (segment (start 114.02 81.228) (end 117.374 84.582) (width 0.25) (layer F.Cu) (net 2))
 (segment (start 138.938 75.184) (end 138.938 82.042) (width 2.2) (layer F.Cu) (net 2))
 (segment (start 138.938 75.152) (end 138.938 75.184) (width 0.3) (layer F.Cu) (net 2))
 (segment (start 124.968 61.182) (end 138.938 75.152) (width 0.3) (layer F.Cu) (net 2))
 (segment (start 92.648 37.128) (end 92.71 37.066) (width 0.25) (layer F.Cu) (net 12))
 (segment (start 92.648 38.628) (end 92.648 37.128) (width 0.25) (layer F.Cu) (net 12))
 (segment (start 92.71 37.066) (end 92.71 36.068) (width 0.25) (layer F.Cu) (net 12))
 (segment (start 92.71 36.068) (end 92.71 36.068) (width 0.25) (layer F.Cu) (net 12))
 (via (at 92.71 36.068) (size 0.8) (drill 0.4) (layers F.Cu B.Cu) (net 12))
 (segment (start 92.71 37.846) (end 92.71 36.068) (width 0.3) (layer B.Cu) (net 12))
 (segment (start 98.552 68.072) (end 99.314 68.834) (width 0.3) (layer B.Cu) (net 12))
 (segment (start 98.552 66.548) (end 98.552 68.072) (width 0.3) (layer B.Cu) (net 12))
 (segment (start 99.314 68.834) (end 103.632 68.834) (width 0.3) (layer B.Cu) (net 12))
 (segment (start 105.156 67.31) (end 105.156 50.292) (width 0.3) (layer B.Cu) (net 12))
 (segment (start 103.632 68.834) (end 105.156 67.31) (width 0.3) (layer B.Cu) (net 12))
 (segment (start 105.156 50.292) (end 92.71 37.846) (width 0.3) (layer B.Cu) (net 12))
 (segment (start 102.616 80.518) (end 102.6635 80.518) (width 0.7) (layer B.Cu) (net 1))
 (segment (start 102.213498 80.518) (end 102.616 80.518) (width 0.7) (layer B.Cu) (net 1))
 (segment (start 102.6635 80.518) (end 102.616 80.518) (width 0.25) (layer F.Cu) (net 1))
 (segment (start 102.5685 80.518) (end 102.616 80.518) (width 0.25) (layer B.Cu) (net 1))
 (segment (start 121.158 68.072) (end 119.634 68.072) (width 2) (layer B.Cu) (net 1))
 (segment (start 115.57 72.136) (end 110.998 72.136) (width 2) (layer B.Cu) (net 1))
 (segment (start 119.634 68.072) (end 115.57 72.136) (width 2) (layer B.Cu) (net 1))
 (segment (start 110.998 72.136) (end 110.998 76.454) (width 2) (layer B.Cu) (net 1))
 (segment (start 110.998 76.454) (end 106.934 80.518) (width 2) (layer B.Cu) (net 1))
 (segment (start 106.934 80.518) (end 101.854 80.518) (width 2) (layer B.Cu) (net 1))
 (segment (start 121.158 62.372) (end 119.968 61.182) (width 0.3) (layer F.Cu) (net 1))
 (segment (start 121.158 68.072) (end 121.158 62.372) (width 0.3) (layer F.Cu) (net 1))
 (segment (start 136.652 68.072) (end 138.938 70.358) (width 2.2) (layer B.Cu) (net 1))
 (segment (start 121.158 68.072) (end 136.652 68.072) (width 2.2) (layer B.Cu) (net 1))
 (segment (start 131.031502 81.16463) (end 131.031502 82.296) (width 0.3) (layer B.Cu) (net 1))
 (segment (start 131.031502 79.810498) (end 131.031502 81.16463) (width 0.3) (layer B.Cu) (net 1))
 (segment (start 138.938 71.904) (end 131.031502 79.810498) (width 0.3) (layer B.Cu) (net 1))
 (segment (start 138.938 70.104) (end 138.938 71.904) (width 0.3) (layer B.Cu) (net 1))
 (segment (start 90.678 53.858) (end 90.648 53.828) (width 0.3) (layer F.Cu) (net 14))
 (segment (start 90.678 60.452) (end 90.678 53.858) (width 0.3) (layer F.Cu) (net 14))
 (segment (start 93.596323 60.452) (end 94.996 61.851677) (width 0.3) (layer F.Cu) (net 14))
 (segment (start 90.678 60.452) (end 93.596323 60.452) (width 0.3) (layer F.Cu) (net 14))
 (segment (start 95.002 61.845677) (end 94.996 61.851677) (width 0.3) (layer F.Cu) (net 14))
 (segment (start 99.697586 61.845677) (end 95.002 61.845677) (width 0.3) (layer F.Cu) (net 14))
 (segment (start 91.53 32.512) (end 91.276 32.258) (width 0.25) (layer F.Cu) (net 17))
 (segment (start 98.648 37.878) (end 98.648 38.628) (width 0.25) (layer F.Cu) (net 17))
 (segment (start 93.472 32.258) (end 94.996 33.782) (width 0.3) (layer F.Cu) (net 17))
 (segment (start 91.276 32.258) (end 93.472 32.258) (width 0.3) (layer F.Cu) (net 17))
 (segment (start 98.648 37.434) (end 98.648 38.628) (width 0.3) (layer F.Cu) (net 17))
 (segment (start 94.996 33.782) (end 98.648 37.434) (width 0.3) (layer F.Cu) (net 17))
 (segment (start 99.06 34.507) (end 100.648 36.095) (width 0.3) (layer F.Cu) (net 18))
 (segment (start 100.648 37.078) (end 100.648 38.628) (width 0.3) (layer F.Cu) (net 18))
 (segment (start 100.648 36.095) (end 100.648 37.078) (width 0.3) (layer F.Cu) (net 18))
 (segment (start 99.06 33.782) (end 99.06 34.507) (width 0.3) (layer F.Cu) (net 18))
 (segment (start 102.616 38.596) (end 102.648 38.628) (width 0.25) (layer F.Cu) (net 19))
 (segment (start 103.124 38.152) (end 102.648 38.628) (width 0.3) (layer F.Cu) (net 19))
 (segment (start 103.124 33.782) (end 103.124 38.152) (width 0.3) (layer F.Cu) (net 19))
 (segment (start 83.566 86.106) (end 87.63 82.042) (width 0.3) (layer F.Cu) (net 20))
 (segment (start 87.63 72.904) (end 90.17 70.364) (width 0.3) (layer F.Cu) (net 20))
 (segment (start 87.63 82.042) (end 87.63 72.904) (width 0.3) (layer F.Cu) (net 20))
 (segment (start 102.648 55.378) (end 102.616 55.41) (width 0.3) (layer F.Cu) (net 20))
 (segment (start 102.648 53.828) (end 102.648 55.378) (width 0.3) (layer F.Cu) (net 20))
 (segment (start 102.616 55.41) (end 102.616 56.388) (width 0.3) (layer F.Cu) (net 20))
 (segment (start 102.616 56.388) (end 102.616 56.388) (width 0.3) (layer F.Cu) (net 20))
 (via (at 102.616 56.388) (size 0.8) (drill 0.4) (layers F.Cu B.Cu) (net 20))
 (segment (start 91.145 70.364) (end 91.151 70.358) (width 0.3) (layer F.Cu) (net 20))
 (segment (start 90.17 70.364) (end 91.145 70.364) (width 0.3) (layer F.Cu) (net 20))
 (segment (start 91.151 70.358) (end 92.456 70.358) (width 0.3) (layer F.Cu) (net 20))
 (segment (start 92.456 70.358) (end 92.456 70.358) (width 0.3) (layer F.Cu) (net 20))
 (via (at 92.456 70.358) (size 0.8) (drill 0.4) (layers F.Cu B.Cu) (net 20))
 (segment (start 92.456 66.548) (end 102.616 56.388) (width 0.3) (layer B.Cu) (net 20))
 (segment (start 92.456 70.358) (end 92.456 66.548) (width 0.3) (layer B.Cu) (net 20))
 (segment (start 84.328 72.898) (end 83.566 73.66) (width 0.3) (layer F.Cu) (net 21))
 (segment (start 84.328 70.488) (end 84.328 72.898) (width 0.3) (layer F.Cu) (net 21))
 (segment (start 100.648 53.828) (end 100.648 56.324) (width 0.3) (layer F.Cu) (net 22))
 (segment (start 100.648 56.324) (end 100.648 56.324) (width 0.3) (layer F.Cu) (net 22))
 (via (at 100.648 56.324) (size 0.8) (drill 0.4) (layers F.Cu B.Cu) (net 22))
 (segment (start 84.328 67.688) (end 84.328 66.963) (width 0.3) (layer F.Cu) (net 22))
 (segment (start 84.328 66.963) (end 84.328 65.532) (width 0.3) (layer F.Cu) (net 22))
 (segment (start 84.328 65.532) (end 84.328 65.532) (width 0.3) (layer F.Cu) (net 22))
 (via (at 84.328 65.532) (size 0.8) (drill 0.4) (layers F.Cu B.Cu) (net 22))
 (segment (start 93.536 56.324) (end 84.328 65.532) (width 0.3) (layer B.Cu) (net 22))
 (segment (start 100.648 56.324) (end 93.536 56.324) (width 0.3) (layer B.Cu) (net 22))
 (segment (start 105.41 73.66) (end 91.186 73.66) (width 0.3) (layer F.Cu) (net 5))
 (segment (start 110.998 68.072) (end 105.41 73.66) (width 0.3) (layer F.Cu) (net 5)))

